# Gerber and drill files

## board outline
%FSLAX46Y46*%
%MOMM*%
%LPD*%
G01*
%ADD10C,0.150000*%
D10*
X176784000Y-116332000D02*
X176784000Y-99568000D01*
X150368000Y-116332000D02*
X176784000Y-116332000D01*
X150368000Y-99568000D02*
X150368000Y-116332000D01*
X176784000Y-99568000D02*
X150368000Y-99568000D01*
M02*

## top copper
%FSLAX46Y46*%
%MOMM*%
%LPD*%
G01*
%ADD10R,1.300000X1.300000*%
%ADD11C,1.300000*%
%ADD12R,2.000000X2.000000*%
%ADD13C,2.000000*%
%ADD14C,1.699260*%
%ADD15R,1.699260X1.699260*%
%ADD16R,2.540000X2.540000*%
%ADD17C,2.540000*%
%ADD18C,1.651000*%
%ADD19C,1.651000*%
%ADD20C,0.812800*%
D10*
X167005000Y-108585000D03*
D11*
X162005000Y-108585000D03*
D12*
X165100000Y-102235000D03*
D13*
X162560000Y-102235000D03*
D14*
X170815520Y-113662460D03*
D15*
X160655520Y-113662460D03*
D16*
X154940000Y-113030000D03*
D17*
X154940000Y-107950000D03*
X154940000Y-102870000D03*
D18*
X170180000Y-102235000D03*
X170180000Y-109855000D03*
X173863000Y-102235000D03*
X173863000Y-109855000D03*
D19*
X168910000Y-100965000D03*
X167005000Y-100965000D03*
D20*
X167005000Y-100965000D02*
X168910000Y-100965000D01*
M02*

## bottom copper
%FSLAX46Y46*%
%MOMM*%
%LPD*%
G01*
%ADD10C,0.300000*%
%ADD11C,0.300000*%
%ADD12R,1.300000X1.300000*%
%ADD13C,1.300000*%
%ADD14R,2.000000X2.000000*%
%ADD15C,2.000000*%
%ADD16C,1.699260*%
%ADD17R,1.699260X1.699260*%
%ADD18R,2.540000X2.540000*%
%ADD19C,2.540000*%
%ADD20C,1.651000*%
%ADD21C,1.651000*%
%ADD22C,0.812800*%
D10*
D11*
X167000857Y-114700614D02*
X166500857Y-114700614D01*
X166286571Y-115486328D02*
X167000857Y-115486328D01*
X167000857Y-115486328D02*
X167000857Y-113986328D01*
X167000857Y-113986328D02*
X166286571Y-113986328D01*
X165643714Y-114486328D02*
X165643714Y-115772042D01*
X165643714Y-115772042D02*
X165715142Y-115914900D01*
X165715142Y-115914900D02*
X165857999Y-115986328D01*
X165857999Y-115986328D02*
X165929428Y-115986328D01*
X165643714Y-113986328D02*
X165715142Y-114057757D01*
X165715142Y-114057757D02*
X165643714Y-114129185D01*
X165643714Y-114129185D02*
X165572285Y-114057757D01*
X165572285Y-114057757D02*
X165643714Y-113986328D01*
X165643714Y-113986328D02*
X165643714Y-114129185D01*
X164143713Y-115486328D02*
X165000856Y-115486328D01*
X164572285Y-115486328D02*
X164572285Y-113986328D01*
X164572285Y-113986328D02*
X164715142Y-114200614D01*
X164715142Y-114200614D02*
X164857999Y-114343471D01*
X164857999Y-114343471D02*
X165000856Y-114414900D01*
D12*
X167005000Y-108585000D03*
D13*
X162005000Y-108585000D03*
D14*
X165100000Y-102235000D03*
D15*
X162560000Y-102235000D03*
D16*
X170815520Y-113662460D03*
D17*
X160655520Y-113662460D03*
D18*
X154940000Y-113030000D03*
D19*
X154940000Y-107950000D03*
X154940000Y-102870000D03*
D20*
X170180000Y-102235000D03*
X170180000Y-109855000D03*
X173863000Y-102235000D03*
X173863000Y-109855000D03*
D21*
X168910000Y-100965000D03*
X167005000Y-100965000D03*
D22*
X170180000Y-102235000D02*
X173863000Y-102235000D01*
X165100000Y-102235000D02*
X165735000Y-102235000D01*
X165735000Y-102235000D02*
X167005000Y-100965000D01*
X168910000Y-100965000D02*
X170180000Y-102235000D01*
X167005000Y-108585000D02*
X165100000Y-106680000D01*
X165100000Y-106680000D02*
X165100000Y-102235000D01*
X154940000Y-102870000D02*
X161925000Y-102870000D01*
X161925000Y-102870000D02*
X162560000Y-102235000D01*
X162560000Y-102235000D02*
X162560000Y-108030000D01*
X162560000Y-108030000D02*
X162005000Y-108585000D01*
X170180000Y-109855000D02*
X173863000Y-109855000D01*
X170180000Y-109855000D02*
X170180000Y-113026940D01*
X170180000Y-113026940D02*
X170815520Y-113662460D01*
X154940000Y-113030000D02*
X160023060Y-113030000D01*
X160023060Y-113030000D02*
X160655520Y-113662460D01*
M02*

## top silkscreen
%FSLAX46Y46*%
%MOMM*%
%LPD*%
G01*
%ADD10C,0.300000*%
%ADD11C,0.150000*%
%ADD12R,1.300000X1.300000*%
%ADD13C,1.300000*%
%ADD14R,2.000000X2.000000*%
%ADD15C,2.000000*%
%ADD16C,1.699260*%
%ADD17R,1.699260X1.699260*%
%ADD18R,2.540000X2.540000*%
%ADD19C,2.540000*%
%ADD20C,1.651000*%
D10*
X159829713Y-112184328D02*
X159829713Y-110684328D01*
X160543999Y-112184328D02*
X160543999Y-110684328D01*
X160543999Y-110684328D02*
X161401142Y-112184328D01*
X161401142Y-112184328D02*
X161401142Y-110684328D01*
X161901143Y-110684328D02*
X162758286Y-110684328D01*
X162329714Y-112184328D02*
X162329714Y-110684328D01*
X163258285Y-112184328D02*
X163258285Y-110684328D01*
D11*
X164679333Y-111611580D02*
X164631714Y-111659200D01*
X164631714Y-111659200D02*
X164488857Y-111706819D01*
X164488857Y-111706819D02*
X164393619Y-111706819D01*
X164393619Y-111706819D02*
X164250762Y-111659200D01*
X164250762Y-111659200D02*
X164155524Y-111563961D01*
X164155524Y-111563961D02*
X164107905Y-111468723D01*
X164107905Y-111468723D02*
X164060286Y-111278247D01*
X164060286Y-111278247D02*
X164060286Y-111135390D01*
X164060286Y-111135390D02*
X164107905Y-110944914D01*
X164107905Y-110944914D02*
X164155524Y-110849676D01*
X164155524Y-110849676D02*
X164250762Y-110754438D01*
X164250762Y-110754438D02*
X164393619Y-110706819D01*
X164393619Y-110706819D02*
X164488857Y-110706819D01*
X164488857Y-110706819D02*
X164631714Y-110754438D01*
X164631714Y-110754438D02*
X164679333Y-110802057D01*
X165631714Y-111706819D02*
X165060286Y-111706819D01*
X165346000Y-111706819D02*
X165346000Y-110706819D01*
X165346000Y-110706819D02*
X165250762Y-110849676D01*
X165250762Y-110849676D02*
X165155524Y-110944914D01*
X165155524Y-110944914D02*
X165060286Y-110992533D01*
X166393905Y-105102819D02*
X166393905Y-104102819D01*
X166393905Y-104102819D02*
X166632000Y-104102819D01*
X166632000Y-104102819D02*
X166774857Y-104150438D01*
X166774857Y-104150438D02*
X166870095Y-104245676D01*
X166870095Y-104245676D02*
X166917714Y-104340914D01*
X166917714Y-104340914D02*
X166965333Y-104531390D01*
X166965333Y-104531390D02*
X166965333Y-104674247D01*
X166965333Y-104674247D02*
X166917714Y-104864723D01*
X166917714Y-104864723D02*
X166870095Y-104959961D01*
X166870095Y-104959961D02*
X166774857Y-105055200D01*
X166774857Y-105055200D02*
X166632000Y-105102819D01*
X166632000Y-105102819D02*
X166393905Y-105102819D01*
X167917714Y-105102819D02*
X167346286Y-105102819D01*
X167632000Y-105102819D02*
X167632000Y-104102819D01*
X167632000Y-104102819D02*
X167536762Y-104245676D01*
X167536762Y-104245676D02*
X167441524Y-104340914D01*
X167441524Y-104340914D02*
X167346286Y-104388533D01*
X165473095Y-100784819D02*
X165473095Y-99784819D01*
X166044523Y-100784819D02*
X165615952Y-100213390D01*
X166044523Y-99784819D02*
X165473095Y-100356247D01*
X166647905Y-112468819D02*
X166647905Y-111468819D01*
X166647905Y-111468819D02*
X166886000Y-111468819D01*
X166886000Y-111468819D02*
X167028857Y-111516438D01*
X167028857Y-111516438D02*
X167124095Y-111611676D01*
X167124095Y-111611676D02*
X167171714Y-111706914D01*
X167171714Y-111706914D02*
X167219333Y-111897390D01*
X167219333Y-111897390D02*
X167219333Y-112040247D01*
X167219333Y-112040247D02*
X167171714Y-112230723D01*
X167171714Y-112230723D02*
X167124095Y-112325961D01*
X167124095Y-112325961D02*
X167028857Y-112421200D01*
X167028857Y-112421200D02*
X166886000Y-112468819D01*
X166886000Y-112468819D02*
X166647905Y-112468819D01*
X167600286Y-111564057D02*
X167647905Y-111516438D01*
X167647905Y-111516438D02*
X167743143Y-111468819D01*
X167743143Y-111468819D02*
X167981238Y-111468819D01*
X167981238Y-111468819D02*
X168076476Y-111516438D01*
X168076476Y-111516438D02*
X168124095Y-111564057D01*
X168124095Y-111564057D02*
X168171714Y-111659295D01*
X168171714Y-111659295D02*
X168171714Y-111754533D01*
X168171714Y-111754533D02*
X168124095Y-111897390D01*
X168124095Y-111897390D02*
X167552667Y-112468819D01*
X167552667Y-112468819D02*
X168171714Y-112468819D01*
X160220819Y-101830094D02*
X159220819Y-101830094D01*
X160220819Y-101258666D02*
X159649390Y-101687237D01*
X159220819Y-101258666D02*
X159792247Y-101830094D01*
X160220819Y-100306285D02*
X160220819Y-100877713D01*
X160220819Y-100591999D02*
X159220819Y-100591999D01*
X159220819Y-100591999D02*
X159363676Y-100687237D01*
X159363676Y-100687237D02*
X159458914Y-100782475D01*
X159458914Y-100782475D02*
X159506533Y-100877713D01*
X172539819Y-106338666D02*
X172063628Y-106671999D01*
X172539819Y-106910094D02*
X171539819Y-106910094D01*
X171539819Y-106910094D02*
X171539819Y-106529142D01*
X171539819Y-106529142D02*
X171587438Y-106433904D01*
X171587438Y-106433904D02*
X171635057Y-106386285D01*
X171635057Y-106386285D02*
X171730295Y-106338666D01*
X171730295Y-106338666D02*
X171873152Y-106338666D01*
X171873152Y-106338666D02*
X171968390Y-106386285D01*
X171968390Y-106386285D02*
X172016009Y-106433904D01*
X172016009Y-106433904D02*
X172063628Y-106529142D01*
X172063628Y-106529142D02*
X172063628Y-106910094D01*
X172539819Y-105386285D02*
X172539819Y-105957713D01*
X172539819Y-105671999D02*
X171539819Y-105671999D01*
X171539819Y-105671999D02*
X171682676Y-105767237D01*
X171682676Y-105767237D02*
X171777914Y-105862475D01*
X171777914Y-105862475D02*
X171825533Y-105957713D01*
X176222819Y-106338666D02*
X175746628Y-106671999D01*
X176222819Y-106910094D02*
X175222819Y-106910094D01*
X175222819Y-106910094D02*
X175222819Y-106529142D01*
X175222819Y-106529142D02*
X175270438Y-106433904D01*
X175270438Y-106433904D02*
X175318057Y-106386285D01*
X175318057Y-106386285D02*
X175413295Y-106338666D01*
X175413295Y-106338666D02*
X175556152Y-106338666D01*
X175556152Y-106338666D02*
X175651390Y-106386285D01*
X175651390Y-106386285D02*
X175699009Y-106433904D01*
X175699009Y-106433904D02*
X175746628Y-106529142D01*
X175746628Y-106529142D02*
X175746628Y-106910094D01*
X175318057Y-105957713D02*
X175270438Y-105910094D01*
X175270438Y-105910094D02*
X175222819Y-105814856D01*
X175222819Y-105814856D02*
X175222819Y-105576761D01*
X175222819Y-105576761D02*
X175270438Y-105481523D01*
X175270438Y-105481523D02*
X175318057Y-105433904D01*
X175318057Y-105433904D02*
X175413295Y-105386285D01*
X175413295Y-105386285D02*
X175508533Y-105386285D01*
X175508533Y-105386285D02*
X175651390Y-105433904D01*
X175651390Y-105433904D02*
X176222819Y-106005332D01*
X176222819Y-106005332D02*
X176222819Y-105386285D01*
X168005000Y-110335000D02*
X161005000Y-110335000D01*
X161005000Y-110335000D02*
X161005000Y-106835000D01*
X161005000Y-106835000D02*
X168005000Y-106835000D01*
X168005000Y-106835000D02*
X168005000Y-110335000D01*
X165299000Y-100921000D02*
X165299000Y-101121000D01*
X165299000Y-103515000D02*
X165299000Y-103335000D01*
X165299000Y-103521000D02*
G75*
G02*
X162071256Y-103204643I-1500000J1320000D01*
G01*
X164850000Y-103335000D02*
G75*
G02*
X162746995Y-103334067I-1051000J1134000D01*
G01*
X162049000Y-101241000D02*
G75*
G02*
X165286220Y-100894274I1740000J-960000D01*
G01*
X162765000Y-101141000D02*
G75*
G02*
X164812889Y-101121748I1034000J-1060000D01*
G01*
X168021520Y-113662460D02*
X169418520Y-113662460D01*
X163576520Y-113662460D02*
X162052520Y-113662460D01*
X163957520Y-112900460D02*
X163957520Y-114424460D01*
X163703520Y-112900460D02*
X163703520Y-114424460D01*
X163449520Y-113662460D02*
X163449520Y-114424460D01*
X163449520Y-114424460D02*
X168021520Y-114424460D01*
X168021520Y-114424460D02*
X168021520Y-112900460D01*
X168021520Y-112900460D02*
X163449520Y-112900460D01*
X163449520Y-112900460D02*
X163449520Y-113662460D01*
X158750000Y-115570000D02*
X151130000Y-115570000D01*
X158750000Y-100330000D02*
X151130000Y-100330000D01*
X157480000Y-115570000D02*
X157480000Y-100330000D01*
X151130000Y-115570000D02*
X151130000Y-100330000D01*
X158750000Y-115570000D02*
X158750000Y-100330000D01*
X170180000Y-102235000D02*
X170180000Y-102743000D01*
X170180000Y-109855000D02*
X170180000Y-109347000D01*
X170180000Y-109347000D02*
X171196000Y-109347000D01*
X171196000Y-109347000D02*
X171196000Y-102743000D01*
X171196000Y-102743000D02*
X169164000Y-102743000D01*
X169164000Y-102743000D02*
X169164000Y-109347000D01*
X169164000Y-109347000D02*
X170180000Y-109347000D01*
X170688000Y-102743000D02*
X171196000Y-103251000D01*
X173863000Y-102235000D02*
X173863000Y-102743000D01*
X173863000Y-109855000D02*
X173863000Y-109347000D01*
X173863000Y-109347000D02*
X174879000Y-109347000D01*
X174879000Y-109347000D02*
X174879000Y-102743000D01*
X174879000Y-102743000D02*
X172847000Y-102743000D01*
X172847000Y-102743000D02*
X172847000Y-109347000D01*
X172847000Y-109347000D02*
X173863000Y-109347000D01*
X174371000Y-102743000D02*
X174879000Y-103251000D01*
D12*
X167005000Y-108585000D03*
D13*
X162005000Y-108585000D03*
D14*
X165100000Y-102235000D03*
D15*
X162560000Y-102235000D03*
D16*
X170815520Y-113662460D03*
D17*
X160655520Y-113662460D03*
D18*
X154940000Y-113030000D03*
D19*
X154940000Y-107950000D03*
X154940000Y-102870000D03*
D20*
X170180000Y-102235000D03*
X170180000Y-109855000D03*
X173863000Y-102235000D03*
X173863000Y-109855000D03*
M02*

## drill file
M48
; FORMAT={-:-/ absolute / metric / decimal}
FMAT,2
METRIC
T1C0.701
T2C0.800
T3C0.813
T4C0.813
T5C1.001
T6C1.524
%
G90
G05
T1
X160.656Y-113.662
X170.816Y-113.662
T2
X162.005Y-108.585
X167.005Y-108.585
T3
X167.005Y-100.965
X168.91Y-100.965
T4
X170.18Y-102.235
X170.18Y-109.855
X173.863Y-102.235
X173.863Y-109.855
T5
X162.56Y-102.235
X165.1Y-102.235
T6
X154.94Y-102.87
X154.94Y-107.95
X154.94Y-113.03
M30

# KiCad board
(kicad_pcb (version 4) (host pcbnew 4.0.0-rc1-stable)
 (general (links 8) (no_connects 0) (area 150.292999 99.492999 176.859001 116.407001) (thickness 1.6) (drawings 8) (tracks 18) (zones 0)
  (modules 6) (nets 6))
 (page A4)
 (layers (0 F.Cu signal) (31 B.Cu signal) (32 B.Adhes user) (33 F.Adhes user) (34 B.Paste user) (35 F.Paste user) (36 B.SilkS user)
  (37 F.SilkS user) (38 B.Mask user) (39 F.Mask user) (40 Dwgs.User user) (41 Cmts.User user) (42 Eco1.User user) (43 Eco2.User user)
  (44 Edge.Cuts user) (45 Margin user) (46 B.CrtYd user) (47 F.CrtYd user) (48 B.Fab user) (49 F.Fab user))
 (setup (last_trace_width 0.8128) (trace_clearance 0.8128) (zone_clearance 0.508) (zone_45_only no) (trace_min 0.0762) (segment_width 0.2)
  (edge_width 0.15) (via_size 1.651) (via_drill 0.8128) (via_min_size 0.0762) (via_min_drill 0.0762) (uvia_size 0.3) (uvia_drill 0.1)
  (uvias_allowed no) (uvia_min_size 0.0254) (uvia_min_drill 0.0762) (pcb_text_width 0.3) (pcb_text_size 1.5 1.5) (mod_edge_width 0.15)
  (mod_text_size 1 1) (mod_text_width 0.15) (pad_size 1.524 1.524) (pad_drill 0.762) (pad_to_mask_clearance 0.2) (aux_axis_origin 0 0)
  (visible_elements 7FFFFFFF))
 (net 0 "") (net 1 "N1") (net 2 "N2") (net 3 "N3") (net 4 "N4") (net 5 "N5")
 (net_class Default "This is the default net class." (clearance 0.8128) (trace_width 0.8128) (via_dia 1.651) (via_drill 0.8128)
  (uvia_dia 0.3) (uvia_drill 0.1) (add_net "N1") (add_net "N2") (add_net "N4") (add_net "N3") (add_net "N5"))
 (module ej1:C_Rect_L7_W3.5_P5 (layer F.Cu) (at 167.005 108.585 180)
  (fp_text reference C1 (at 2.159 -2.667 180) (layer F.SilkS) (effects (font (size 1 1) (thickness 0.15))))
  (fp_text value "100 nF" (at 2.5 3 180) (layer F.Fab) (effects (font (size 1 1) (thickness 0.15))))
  (fp_line (start -1 -1.75) (end 6 -1.75) (layer F.SilkS) (width 0.15))
  (fp_line (start 6 -1.75) (end 6 1.75) (layer F.SilkS) (width 0.15))
  (fp_line (start 6 1.75) (end -1 1.75) (layer F.SilkS) (width 0.15))
  (fp_line (start -1 1.75) (end -1 -1.75) (layer F.SilkS) (width 0.15))
  (pad 1 thru_hole rect (at 0 0 180) (size 1.3 1.3) (drill 0.8) (layers *.Cu *.Mask F.SilkS) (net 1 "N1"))
  (pad 2 thru_hole circle (at 5 0 180) (size 1.3 1.3) (drill 0.8) (layers *.Cu *.Mask F.SilkS) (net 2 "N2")))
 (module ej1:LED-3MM (layer F.Cu) (at 165.1 102.235 180)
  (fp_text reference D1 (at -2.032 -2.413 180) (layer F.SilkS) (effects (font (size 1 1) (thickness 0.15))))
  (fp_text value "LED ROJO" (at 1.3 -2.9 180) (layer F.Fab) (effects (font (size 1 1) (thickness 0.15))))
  (fp_line (start -0.199 1.314) (end -0.199 1.114) (layer F.SilkS) (width 0.15))
  (fp_line (start -0.199 -1.28) (end -0.199 -1.1) (layer F.SilkS) (width 0.15))
  (fp_arc (start 1.301 0.034) (end -0.199 -1.286) (angle 108.5) (layer F.SilkS) (width 0.15))
  (fp_arc (start 1.301 0.034) (end 0.25 -1.1) (angle 85.7) (layer F.SilkS) (width 0.15))
  (fp_arc (start 1.311 0.034) (end 3.051 0.994) (angle 110) (layer F.SilkS) (width 0.15))
  (fp_arc (start 1.301 0.034) (end 2.335 1.094) (angle 87.5) (layer F.SilkS) (width 0.15))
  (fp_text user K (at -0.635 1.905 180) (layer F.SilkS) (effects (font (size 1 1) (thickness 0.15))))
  (pad 1 thru_hole rect (at 0 0 270) (size 2 2) (drill 1.00076) (layers *.Cu *.Mask F.SilkS) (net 1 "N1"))
  (pad 2 thru_hole circle (at 2.54 0 180) (size 2 2) (drill 1.00076) (layers *.Cu *.Mask F.SilkS) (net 2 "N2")))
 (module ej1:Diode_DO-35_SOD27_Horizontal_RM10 (layer F.Cu) (at 160.655 113.665)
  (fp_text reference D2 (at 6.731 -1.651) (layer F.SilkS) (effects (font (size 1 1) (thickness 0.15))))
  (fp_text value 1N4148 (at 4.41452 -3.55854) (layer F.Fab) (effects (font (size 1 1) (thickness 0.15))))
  (fp_line (start 7.36652 -0.00254) (end 8.76352 -0.00254) (layer F.SilkS) (width 0.15))
  (fp_line (start 2.92152 -0.00254) (end 1.39752 -0.00254) (layer F.SilkS) (width 0.15))
  (fp_line (start 3.30252 -0.76454) (end 3.30252 0.75946) (layer F.SilkS) (width 0.15))
  (fp_line (start 3.04852 -0.76454) (end 3.04852 0.75946) (layer F.SilkS) (width 0.15))
  (fp_line (start 2.79452 -0.00254) (end 2.79452 0.75946) (layer F.SilkS) (width 0.15))
  (fp_line (start 2.79452 0.75946) (end 7.36652 0.75946) (layer F.SilkS) (width 0.15))
  (fp_line (start 7.36652 0.75946) (end 7.36652 -0.76454) (layer F.SilkS) (width 0.15))
  (fp_line (start 7.36652 -0.76454) (end 2.79452 -0.76454) (layer F.SilkS) (width 0.15))
  (fp_line (start 2.79452 -0.76454) (end 2.79452 -0.00254) (layer F.SilkS) (width 0.15))
  (pad 2 thru_hole circle (at 10.16052 -0.00254 180) (size 1.69926 1.69926) (drill 0.70104) (layers *.Cu *.Mask F.SilkS) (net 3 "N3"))
  (pad 1 thru_hole rect (at 0.00052 -0.00254 180) (size 1.69926 1.69926) (drill 0.70104) (layers *.Cu *.Mask F.SilkS) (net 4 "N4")))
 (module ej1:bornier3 (layer F.Cu) (at 154.94 107.95 90)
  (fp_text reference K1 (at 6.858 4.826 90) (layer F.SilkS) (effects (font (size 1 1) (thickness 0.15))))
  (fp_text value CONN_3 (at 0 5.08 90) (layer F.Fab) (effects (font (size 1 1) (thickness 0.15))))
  (fp_line (start -7.62 3.81) (end -7.62 -3.81) (layer F.SilkS) (width 0.15))
  (fp_line (start 7.62 3.81) (end 7.62 -3.81) (layer F.SilkS) (width 0.15))
  (fp_line (start -7.62 2.54) (end 7.62 2.54) (layer F.SilkS) (width 0.15))
  (fp_line (start -7.62 -3.81) (end 7.62 -3.81) (layer F.SilkS) (width 0.15))
  (fp_line (start -7.62 3.81) (end 7.62 3.81) (layer F.SilkS) (width 0.15))
  (pad 1 thru_hole rect (at -5.08 0 90) (size 2.54 2.54) (drill 1.524) (layers *.Cu *.Mask F.SilkS) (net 4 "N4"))
  (pad 2 thru_hole circle (at 0 0 90) (size 2.54 2.54) (drill 1.524) (layers *.Cu *.Mask F.SilkS) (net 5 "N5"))
  (pad 3 thru_hole circle (at 5.08 0 90) (size 2.54 2.54) (drill 1.524) (layers *.Cu *.Mask F.SilkS) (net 2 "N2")))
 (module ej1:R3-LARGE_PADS (layer F.Cu) (at 170.18 106.045 270)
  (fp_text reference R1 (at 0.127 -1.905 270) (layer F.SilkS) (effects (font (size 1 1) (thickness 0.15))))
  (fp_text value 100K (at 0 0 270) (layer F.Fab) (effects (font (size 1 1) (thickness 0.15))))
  (fp_line (start -3.81 0) (end -3.302 0) (layer F.SilkS) (width 0.15))
  (fp_line (start 3.81 0) (end 3.302 0) (layer F.SilkS) (width 0.15))
  (fp_line (start 3.302 0) (end 3.302 -1.016) (layer F.SilkS) (width 0.15))
  (fp_line (start 3.302 -1.016) (end -3.302 -1.016) (layer F.SilkS) (width 0.15))
  (fp_line (start -3.302 -1.016) (end -3.302 1.016) (layer F.SilkS) (width 0.15))
  (fp_line (start -3.302 1.016) (end 3.302 1.016) (layer F.SilkS) (width 0.15))
  (fp_line (start 3.302 1.016) (end 3.302 0) (layer F.SilkS) (width 0.15))
  (fp_line (start -3.302 -0.508) (end -2.794 -1.016) (layer F.SilkS) (width 0.15))
  (pad 1 thru_hole circle (at -3.81 0 270) (size 1.651 1.651) (drill 0.8128) (layers *.Cu *.Mask F.SilkS) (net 1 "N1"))
  (pad 2 thru_hole circle (at 3.81 0 270) (size 1.651 1.651) (drill 0.8128) (layers *.Cu *.Mask F.SilkS) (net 3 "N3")))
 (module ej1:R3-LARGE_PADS (layer F.Cu) (at 173.863 106.045 270)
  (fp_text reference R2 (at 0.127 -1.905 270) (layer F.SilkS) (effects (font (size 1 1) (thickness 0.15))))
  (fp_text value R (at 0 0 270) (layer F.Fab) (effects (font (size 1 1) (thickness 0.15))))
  (fp_line (start -3.81 0) (end -3.302 0) (layer F.SilkS) (width 0.15))
  (fp_line (start 3.81 0) (end 3.302 0) (layer F.SilkS) (width 0.15))
  (fp_line (start 3.302 0) (end 3.302 -1.016) (layer F.SilkS) (width 0.15))
  (fp_line (start 3.302 -1.016) (end -3.302 -1.016) (layer F.SilkS) (width 0.15))
  (fp_line (start -3.302 -1.016) (end -3.302 1.016) (layer F.SilkS) (width 0.15))
  (fp_line (start -3.302 1.016) (end 3.302 1.016) (layer F.SilkS) (width 0.15))
  (fp_line (start 3.302 1.016) (end 3.302 0) (layer F.SilkS) (width 0.15))
  (fp_line (start -3.302 -0.508) (end -2.794 -1.016) (layer F.SilkS) (width 0.15))
  (pad 1 thru_hole circle (at -3.81 0 270) (size 1.651 1.651) (drill 0.8128) (layers *.Cu *.Mask F.SilkS) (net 1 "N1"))
  (pad 2 thru_hole circle (at 3.81 0 270) (size 1.651 1.651) (drill 0.8128) (layers *.Cu *.Mask F.SilkS) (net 3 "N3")))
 (gr_line (start 176.784 116.332) (end 176.784 99.568) (angle 90) (layer Edge.Cuts) (width 0.15))
 (gr_line (start 150.368 116.332) (end 176.784 116.332) (angle 90) (layer Edge.Cuts) (width 0.15))
 (gr_line (start 150.368 99.568) (end 150.368 116.332) (angle 90) (layer Edge.Cuts) (width 0.15))
 (gr_line (start 176.784 99.568) (end 150.368 99.568) (angle 90) (layer Edge.Cuts) (width 0.15))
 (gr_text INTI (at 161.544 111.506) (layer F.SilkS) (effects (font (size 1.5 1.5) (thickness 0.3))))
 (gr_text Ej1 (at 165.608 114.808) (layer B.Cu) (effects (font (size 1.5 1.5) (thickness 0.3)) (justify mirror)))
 (segment (start 170.18 102.235) (end 173.863 102.235) (width 0.8128) (layer B.Cu) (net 1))
 (segment (start 165.1 102.235) (end 165.735 102.235) (width 0.8128) (layer B.Cu) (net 1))
 (segment (start 165.735 102.235) (end 167.005 100.965) (width 0.8128) (layer B.Cu) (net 1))
 (segment (start 168.91 100.965) (end 170.18 102.235) (width 0.8128) (layer B.Cu) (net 1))
 (via (at 168.91 100.965) (size 1.651) (drill 0.8128) (layers F.Cu B.Cu) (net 1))
 (segment (start 167.005 100.965) (end 168.91 100.965) (width 0.8128) (layer F.Cu) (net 1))
 (via (at 167.005 100.965) (size 1.651) (drill 0.8128) (layers F.Cu B.Cu) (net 1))
 (segment (start 167.005 108.585) (end 165.1 106.68) (width 0.8128) (layer B.Cu) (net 1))
 (segment (start 165.1 106.68) (end 165.1 102.235) (width 0.8128) (layer B.Cu) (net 1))
 (segment (start 154.94 102.87) (end 161.925 102.87) (width 0.8128) (layer B.Cu) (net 2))
 (segment (start 161.925 102.87) (end 162.56 102.235) (width 0.8128) (layer B.Cu) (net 2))
 (segment (start 162.56 102.235) (end 162.56 108.03) (width 0.8128) (layer B.Cu) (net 2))
 (segment (start 162.56 108.03) (end 162.005 108.585) (width 0.8128) (layer B.Cu) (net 2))
 (segment (start 170.18 109.855) (end 173.863 109.855) (width 0.8128) (layer B.Cu) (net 3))
 (segment (start 170.18 109.855) (end 170.18 113.02694) (width 0.8128) (layer B.Cu) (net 3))
 (segment (start 170.18 113.02694) (end 170.81552 113.66246) (width 0.8128) (layer B.Cu) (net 3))
 (segment (start 154.94 113.03) (end 160.02306 113.03) (width 0.8128) (layer B.Cu) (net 4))
 (segment (start 160.02306 113.03) (end 160.65552 113.66246) (width 0.8128) (layer B.Cu) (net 4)))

